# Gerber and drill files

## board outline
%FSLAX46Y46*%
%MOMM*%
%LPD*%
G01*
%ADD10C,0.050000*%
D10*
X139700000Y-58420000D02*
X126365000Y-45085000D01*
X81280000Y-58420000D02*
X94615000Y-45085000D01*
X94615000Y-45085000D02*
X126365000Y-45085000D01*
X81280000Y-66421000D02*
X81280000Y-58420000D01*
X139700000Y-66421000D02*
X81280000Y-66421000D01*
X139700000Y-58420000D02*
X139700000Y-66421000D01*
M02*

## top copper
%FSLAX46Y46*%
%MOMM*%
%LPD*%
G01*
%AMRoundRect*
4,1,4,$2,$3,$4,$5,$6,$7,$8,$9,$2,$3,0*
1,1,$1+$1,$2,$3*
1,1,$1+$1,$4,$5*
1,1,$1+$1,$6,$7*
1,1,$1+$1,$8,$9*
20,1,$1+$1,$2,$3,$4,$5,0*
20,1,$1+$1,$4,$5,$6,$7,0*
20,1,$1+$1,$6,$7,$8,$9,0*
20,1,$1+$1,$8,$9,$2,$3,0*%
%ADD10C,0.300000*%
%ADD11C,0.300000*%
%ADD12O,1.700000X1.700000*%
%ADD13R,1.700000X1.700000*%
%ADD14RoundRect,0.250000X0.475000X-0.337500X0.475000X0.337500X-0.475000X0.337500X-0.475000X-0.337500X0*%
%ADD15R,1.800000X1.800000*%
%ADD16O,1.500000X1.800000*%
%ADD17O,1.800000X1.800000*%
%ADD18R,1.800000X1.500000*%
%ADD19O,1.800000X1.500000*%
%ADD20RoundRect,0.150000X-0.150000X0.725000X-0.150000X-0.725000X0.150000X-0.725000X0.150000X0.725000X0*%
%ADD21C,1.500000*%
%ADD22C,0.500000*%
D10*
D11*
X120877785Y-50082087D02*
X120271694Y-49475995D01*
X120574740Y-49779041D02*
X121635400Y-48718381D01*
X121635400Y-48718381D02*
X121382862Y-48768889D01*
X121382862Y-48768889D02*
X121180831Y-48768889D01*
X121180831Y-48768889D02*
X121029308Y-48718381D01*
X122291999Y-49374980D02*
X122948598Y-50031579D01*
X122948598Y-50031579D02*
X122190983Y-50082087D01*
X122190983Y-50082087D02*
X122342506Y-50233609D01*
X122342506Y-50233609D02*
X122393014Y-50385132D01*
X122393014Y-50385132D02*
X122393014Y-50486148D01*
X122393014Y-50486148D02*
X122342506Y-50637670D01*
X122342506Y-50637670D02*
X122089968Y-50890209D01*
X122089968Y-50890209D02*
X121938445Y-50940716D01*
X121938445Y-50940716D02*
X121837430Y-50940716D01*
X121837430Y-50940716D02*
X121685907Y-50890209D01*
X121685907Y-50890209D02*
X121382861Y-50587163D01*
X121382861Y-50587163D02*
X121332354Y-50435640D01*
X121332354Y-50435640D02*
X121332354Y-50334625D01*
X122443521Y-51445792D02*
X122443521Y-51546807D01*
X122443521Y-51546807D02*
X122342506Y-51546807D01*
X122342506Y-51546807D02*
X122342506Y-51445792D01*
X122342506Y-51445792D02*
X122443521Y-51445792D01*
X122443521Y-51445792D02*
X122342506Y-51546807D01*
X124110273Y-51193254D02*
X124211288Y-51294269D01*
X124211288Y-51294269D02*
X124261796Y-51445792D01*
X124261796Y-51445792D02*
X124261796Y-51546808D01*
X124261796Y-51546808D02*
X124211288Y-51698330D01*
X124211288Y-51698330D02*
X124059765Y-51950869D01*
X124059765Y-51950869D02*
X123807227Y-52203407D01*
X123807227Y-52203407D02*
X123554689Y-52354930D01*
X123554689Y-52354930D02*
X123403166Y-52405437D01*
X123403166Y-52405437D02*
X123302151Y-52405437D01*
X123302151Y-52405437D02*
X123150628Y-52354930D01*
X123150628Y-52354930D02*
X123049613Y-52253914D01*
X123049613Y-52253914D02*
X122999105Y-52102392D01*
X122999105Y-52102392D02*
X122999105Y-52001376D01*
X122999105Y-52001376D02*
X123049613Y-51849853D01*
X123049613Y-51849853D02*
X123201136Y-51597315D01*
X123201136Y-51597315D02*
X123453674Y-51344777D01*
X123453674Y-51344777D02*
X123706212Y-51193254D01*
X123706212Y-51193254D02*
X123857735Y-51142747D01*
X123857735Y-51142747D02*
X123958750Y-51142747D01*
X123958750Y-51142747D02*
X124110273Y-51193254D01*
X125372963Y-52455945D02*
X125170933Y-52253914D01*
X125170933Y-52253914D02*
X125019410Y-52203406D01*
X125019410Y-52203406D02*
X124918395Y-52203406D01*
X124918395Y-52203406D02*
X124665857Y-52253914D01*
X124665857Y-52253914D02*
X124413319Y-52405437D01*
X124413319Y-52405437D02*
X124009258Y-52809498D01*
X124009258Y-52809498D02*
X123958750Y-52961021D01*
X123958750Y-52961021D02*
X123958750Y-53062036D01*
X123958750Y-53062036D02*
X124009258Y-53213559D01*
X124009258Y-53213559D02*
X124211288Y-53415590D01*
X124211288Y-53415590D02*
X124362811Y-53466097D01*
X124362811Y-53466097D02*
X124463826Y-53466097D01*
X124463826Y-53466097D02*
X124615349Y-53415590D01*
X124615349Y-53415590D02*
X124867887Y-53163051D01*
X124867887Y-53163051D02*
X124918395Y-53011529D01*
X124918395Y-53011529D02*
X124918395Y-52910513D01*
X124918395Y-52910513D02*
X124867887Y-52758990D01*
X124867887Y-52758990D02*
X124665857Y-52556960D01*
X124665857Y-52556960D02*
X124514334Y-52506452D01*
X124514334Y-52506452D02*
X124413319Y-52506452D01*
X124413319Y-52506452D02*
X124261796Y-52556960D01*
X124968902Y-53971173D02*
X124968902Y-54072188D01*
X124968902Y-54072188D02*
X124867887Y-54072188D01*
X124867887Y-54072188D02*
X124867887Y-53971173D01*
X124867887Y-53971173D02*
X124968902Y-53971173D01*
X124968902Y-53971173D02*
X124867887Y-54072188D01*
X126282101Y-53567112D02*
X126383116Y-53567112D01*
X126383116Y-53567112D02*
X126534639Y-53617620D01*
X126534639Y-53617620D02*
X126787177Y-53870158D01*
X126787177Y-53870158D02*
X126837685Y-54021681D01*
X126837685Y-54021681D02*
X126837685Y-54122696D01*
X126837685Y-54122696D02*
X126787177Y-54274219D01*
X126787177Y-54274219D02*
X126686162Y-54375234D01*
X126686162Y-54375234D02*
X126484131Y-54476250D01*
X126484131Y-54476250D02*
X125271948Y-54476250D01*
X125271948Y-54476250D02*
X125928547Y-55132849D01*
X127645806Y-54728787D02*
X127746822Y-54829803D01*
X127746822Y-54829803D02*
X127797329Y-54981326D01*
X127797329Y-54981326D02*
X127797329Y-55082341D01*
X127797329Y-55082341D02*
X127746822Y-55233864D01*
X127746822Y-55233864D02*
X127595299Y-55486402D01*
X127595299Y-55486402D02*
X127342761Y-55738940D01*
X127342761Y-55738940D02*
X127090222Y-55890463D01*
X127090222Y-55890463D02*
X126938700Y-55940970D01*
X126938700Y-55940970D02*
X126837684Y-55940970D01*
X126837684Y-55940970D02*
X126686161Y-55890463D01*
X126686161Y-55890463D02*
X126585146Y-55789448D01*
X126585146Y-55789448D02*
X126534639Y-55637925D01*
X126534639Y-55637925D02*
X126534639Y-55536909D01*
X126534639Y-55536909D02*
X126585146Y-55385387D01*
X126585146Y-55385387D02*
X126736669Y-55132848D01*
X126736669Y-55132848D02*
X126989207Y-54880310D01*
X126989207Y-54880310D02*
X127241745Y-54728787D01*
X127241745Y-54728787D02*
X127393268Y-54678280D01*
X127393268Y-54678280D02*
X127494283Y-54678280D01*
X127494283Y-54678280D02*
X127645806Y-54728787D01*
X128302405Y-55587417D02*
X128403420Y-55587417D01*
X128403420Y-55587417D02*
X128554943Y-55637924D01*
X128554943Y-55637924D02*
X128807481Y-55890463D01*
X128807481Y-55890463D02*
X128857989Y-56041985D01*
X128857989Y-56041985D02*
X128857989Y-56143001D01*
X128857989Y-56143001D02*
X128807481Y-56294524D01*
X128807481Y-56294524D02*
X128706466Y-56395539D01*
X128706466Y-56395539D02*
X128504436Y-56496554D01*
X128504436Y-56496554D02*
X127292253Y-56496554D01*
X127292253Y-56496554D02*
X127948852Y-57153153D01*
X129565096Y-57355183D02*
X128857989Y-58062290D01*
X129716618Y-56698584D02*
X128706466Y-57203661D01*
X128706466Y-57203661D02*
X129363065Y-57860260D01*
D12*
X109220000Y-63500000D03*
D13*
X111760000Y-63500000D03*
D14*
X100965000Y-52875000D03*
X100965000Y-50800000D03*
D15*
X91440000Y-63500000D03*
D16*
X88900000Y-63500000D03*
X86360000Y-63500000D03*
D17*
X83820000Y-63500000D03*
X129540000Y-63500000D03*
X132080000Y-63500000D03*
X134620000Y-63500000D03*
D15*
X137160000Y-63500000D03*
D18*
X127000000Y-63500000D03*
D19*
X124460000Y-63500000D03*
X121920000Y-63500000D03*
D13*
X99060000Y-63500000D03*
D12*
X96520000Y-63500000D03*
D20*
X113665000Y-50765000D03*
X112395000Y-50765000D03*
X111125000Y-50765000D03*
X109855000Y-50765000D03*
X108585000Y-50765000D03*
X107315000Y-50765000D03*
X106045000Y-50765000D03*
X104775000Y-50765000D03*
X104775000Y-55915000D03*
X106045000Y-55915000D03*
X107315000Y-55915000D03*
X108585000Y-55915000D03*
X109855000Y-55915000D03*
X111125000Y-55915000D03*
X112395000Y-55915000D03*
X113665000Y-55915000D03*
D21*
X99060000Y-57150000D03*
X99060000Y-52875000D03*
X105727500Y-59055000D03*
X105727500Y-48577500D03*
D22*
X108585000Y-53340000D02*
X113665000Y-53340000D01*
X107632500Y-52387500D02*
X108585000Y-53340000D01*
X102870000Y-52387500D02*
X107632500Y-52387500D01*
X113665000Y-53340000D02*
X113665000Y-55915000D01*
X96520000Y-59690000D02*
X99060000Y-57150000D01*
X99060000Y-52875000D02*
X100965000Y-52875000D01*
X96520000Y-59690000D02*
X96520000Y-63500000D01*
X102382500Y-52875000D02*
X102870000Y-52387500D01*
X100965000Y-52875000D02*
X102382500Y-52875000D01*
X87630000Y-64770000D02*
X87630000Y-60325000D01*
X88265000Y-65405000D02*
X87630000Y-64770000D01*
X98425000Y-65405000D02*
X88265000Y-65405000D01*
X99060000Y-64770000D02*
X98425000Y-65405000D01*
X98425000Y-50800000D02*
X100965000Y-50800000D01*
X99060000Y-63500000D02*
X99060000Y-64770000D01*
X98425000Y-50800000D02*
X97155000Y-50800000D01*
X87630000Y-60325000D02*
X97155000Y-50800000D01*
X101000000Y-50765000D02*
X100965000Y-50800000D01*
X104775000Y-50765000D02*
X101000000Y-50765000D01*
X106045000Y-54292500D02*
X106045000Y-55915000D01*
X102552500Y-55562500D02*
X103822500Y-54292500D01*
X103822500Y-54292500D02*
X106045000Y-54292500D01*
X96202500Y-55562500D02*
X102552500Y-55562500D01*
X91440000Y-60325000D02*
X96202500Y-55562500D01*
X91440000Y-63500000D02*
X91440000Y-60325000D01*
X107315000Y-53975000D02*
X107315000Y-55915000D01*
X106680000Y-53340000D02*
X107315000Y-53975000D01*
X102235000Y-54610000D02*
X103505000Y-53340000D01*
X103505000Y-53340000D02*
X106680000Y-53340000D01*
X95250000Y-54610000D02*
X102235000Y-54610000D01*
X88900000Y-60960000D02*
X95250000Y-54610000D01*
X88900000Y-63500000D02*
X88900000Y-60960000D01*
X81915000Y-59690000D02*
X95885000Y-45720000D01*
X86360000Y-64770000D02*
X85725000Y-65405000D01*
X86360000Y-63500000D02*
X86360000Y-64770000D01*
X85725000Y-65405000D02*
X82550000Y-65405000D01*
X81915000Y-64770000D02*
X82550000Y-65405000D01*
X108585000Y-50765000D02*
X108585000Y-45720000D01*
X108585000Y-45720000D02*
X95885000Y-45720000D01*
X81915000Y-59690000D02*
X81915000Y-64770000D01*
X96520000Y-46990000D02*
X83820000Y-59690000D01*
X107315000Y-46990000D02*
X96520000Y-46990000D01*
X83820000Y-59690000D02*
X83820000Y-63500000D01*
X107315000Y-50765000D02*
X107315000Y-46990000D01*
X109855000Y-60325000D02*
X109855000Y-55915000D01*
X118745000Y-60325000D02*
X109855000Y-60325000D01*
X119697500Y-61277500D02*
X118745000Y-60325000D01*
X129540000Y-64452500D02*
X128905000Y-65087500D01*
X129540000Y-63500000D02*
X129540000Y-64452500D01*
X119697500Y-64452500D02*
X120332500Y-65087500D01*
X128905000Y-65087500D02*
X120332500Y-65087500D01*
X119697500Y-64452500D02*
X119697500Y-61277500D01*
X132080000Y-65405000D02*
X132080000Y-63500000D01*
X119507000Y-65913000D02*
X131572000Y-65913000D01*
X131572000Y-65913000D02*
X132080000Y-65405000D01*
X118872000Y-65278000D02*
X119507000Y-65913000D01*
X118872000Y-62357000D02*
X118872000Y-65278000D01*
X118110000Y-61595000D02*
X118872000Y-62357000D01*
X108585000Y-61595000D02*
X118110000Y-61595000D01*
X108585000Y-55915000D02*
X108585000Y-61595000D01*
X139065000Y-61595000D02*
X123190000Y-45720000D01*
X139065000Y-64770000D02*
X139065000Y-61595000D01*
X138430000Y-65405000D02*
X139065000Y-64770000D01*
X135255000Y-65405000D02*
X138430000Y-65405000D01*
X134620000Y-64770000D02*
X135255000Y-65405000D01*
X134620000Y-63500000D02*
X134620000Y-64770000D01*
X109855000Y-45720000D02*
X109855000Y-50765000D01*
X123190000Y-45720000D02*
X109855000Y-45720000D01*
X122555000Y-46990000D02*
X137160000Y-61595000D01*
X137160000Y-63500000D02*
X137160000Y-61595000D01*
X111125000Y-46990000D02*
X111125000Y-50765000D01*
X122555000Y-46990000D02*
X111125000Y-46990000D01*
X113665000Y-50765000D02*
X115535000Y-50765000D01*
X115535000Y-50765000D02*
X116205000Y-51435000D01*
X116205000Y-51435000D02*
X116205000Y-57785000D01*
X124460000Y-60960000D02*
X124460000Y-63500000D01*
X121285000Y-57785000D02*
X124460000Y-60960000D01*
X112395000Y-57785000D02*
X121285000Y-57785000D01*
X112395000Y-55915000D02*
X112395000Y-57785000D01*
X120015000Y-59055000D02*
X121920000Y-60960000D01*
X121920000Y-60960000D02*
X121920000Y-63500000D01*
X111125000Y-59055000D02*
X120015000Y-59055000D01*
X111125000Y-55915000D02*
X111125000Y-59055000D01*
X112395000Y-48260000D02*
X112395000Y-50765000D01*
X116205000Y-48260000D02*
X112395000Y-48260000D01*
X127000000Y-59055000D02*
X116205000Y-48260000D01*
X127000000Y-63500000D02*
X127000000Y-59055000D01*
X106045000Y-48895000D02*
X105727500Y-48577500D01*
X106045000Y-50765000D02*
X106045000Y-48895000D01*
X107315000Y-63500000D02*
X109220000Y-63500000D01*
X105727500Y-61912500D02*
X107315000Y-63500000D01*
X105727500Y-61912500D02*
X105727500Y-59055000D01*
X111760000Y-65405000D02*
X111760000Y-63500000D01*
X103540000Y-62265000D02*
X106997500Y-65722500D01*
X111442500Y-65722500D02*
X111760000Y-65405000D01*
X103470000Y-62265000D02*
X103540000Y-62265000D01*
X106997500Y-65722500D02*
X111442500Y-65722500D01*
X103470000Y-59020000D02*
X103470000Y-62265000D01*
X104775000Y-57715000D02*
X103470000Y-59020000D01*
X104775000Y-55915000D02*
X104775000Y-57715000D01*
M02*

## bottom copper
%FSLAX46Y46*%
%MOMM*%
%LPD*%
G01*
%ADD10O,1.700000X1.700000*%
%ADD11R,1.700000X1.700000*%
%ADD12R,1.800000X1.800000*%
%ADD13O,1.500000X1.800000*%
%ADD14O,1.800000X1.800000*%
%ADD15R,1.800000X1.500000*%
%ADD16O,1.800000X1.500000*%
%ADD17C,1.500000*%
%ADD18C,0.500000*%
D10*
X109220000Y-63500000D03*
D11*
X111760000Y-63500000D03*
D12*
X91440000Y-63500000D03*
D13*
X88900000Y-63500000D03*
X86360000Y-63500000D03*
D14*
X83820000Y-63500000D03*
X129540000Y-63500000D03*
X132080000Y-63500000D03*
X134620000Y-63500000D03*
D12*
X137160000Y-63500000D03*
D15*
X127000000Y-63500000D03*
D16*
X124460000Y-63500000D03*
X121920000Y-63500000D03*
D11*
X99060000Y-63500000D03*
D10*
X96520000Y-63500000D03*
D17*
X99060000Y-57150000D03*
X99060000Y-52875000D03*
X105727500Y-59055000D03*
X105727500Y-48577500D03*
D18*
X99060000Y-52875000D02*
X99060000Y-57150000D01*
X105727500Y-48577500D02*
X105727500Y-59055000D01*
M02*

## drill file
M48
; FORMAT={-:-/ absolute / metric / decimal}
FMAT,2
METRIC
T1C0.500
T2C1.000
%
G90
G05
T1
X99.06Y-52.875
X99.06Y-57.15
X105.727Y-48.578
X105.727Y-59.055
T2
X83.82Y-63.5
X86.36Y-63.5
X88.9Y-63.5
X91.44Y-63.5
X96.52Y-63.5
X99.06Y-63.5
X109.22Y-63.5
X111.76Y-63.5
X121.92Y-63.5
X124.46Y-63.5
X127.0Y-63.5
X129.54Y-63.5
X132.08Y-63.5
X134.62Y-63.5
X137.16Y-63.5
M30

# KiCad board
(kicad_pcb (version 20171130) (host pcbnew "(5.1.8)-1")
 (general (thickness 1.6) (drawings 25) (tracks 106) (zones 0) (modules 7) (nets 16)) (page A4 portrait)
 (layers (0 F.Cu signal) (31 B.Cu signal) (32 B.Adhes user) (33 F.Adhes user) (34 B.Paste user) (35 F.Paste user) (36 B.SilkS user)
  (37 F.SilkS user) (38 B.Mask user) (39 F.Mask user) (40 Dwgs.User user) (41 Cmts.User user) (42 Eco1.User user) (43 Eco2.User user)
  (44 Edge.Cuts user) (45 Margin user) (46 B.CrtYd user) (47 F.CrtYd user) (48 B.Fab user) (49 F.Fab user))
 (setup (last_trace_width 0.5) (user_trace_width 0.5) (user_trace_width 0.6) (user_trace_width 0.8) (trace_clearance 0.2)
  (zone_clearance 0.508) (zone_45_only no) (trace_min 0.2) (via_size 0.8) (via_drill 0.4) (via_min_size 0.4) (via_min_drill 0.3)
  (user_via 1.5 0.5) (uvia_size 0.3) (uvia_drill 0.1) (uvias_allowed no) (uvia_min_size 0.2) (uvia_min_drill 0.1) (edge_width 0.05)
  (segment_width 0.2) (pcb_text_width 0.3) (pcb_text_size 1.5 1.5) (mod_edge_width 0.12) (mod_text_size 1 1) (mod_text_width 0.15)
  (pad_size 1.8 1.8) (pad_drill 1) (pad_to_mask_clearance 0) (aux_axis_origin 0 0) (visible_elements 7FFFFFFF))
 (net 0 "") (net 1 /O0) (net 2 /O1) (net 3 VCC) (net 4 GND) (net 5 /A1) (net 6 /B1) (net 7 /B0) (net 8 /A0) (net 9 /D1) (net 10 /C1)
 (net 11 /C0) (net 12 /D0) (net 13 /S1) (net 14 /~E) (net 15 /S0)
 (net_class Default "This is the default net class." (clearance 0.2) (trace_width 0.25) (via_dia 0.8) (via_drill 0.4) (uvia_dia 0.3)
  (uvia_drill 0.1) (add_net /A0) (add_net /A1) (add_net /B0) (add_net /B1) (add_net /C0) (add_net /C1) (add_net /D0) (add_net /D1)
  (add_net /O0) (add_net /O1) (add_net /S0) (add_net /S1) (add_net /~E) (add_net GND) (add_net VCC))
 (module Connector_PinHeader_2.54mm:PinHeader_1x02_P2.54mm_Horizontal (layer F.Cu) (at 111.76 63.5 270)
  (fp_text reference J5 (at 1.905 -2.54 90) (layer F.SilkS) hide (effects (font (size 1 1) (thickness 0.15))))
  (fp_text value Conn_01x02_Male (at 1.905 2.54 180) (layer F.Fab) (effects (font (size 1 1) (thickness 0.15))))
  (pad 2 thru_hole oval (at 0 2.54 270) (size 1.7 1.7) (drill 1) (layers *.Cu *.Mask) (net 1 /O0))
  (pad 1 thru_hole rect (at 0 0 270) (size 1.7 1.7) (drill 1) (layers *.Cu *.Mask) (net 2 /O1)))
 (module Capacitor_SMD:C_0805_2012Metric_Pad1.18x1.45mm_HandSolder (layer F.Cu) (at 100.965 51.8375 90)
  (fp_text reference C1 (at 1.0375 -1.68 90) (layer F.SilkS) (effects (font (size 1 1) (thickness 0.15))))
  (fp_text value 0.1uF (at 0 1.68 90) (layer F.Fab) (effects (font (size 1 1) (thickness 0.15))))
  (pad 1 smd roundrect (at -1.0375 0 90) (size 1.175 1.45) (layers F.Cu F.Paste F.Mask) (roundrect_rratio 0.2127659574468085) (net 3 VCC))
  (pad 2 smd roundrect (at 1.0375 0 90) (size 1.175 1.45) (layers F.Cu F.Paste F.Mask) (roundrect_rratio 0.2127659574468085) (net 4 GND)))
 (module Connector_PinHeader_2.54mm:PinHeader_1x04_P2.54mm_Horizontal (layer F.Cu) (at 91.44 63.5 270)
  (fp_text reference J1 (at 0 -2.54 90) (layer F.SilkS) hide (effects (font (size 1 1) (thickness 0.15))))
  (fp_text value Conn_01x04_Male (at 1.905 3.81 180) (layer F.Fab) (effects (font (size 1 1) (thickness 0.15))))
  (pad 1 thru_hole rect (at 0 0 270) (size 1.8 1.8) (drill 1) (layers *.Cu *.Mask) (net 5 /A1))
  (pad 2 thru_hole oval (at 0 2.54 270) (size 1.8 1.5) (drill 1) (layers *.Cu *.Mask) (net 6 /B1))
  (pad 3 thru_hole oval (at 0 5.08 270) (size 1.8 1.5) (drill 1) (layers *.Cu *.Mask) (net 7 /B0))
  (pad 4 thru_hole oval (at 0 7.62 270) (size 1.8 1.8) (drill 1) (layers *.Cu *.Mask) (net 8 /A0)))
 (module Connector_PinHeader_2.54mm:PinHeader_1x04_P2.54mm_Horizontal (layer F.Cu) (at 137.16 63.5 270)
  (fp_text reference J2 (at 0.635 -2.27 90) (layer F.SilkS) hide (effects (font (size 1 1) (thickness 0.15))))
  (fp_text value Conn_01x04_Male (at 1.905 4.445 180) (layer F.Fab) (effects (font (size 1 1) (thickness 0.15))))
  (pad 4 thru_hole oval (at 0 7.62 270) (size 1.8 1.8) (drill 1) (layers *.Cu *.Mask) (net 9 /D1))
  (pad 3 thru_hole oval (at 0 5.08 270) (size 1.8 1.8) (drill 1) (layers *.Cu *.Mask) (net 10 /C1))
  (pad 2 thru_hole oval (at 0 2.54 270) (size 1.8 1.8) (drill 1) (layers *.Cu *.Mask) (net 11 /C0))
  (pad 1 thru_hole rect (at 0 0 270) (size 1.8 1.8) (drill 1) (layers *.Cu *.Mask) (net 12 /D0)))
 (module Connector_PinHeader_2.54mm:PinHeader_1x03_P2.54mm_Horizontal (layer F.Cu) (at 127 63.5 270)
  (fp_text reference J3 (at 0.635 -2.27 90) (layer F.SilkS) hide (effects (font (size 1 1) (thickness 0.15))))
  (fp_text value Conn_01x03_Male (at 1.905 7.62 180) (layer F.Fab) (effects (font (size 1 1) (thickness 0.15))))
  (pad 1 thru_hole rect (at 0 0 270) (size 1.5 1.8) (drill 1) (layers *.Cu *.Mask) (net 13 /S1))
  (pad 2 thru_hole oval (at 0 2.54 270) (size 1.5 1.8) (drill 1) (layers *.Cu *.Mask) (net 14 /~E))
  (pad 3 thru_hole oval (at 0 5.08 270) (size 1.5 1.8) (drill 1) (layers *.Cu *.Mask) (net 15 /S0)))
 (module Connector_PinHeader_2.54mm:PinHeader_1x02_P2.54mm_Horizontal (layer F.Cu) (at 99.06 63.5 270)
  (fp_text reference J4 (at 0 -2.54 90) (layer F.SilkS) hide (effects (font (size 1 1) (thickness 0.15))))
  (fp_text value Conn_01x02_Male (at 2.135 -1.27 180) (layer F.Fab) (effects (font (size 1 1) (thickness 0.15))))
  (pad 1 thru_hole rect (at 0 0 270) (size 1.7 1.7) (drill 1) (layers *.Cu *.Mask) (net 4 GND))
  (pad 2 thru_hole oval (at 0 2.54 270) (size 1.7 1.7) (drill 1) (layers *.Cu *.Mask) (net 3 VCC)))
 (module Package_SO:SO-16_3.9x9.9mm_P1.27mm (layer F.Cu) (at 109.22 53.34 270)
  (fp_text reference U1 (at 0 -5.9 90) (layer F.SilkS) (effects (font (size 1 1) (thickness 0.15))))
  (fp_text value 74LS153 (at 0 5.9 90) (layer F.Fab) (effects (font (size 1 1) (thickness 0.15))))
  (pad 1 smd roundrect (at -2.575 -4.445 270) (size 1.75 0.6) (layers F.Cu F.Paste F.Mask) (roundrect_rratio 0.25) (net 14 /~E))
  (pad 2 smd roundrect (at -2.575 -3.175 270) (size 1.75 0.6) (layers F.Cu F.Paste F.Mask) (roundrect_rratio 0.25) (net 13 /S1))
  (pad 3 smd roundrect (at -2.575 -1.905 270) (size 1.75 0.6) (layers F.Cu F.Paste F.Mask) (roundrect_rratio 0.25) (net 12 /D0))
  (pad 4 smd roundrect (at -2.575 -0.635 270) (size 1.75 0.6) (layers F.Cu F.Paste F.Mask) (roundrect_rratio 0.25) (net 11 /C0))
  (pad 5 smd roundrect (at -2.575 0.635 270) (size 1.75 0.6) (layers F.Cu F.Paste F.Mask) (roundrect_rratio 0.25) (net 7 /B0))
  (pad 6 smd roundrect (at -2.575 1.905 270) (size 1.75 0.6) (layers F.Cu F.Paste F.Mask) (roundrect_rratio 0.25) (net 8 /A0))
  (pad 7 smd roundrect (at -2.575 3.175 270) (size 1.75 0.6) (layers F.Cu F.Paste F.Mask) (roundrect_rratio 0.25) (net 1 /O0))
  (pad 8 smd roundrect (at -2.575 4.445 270) (size 1.75 0.6) (layers F.Cu F.Paste F.Mask) (roundrect_rratio 0.25) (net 4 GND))
  (pad 9 smd roundrect (at 2.575 4.445 270) (size 1.75 0.6) (layers F.Cu F.Paste F.Mask) (roundrect_rratio 0.25) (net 2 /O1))
  (pad 10 smd roundrect (at 2.575 3.175 270) (size 1.75 0.6) (layers F.Cu F.Paste F.Mask) (roundrect_rratio 0.25) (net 5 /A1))
  (pad 11 smd roundrect (at 2.575 1.905 270) (size 1.75 0.6) (layers F.Cu F.Paste F.Mask) (roundrect_rratio 0.25) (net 6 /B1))
  (pad 12 smd roundrect (at 2.575 0.635 270) (size 1.75 0.6) (layers F.Cu F.Paste F.Mask) (roundrect_rratio 0.25) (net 10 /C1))
  (pad 13 smd roundrect (at 2.575 -0.635 270) (size 1.75 0.6) (layers F.Cu F.Paste F.Mask) (roundrect_rratio 0.25) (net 9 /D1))
  (pad 14 smd roundrect (at 2.575 -1.905 270) (size 1.75 0.6) (layers F.Cu F.Paste F.Mask) (roundrect_rratio 0.25) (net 15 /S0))
  (pad 15 smd roundrect (at 2.575 -3.175 270) (size 1.75 0.6) (layers F.Cu F.Paste F.Mask) (roundrect_rratio 0.25) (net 14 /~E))
  (pad 16 smd roundrect (at 2.575 -4.445 270) (size 1.75 0.6) (layers F.Cu F.Paste F.Mask) (roundrect_rratio 0.25) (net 3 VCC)))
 (gr_line (start 139.7 58.42) (end 126.365 45.085) (layer Edge.Cuts) (width 0.05))
 (gr_line (start 81.28 58.42) (end 94.615 45.085) (layer Edge.Cuts) (width 0.05))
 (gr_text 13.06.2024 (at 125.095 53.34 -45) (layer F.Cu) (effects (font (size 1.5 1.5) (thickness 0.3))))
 (gr_line (start 94.615 45.085) (end 126.365 45.085) (layer Edge.Cuts) (width 0.05))
 (gr_line (start 81.28 66.421) (end 81.28 58.42) (layer Edge.Cuts) (width 0.05))
 (gr_line (start 139.7 66.421) (end 81.28 66.421) (layer Edge.Cuts) (width 0.05))
 (gr_line (start 139.7 58.42) (end 139.7 66.421) (layer Edge.Cuts) (width 0.05))
 (segment (start 108.585 53.34) (end 113.665 53.34) (width 0.5) (layer F.Cu) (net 3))
 (segment (start 107.6325 52.3875) (end 108.585 53.34) (width 0.5) (layer F.Cu) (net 3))
 (segment (start 102.87 52.3875) (end 107.6325 52.3875) (width 0.5) (layer F.Cu) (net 3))
 (via (at 99.06 57.15) (size 1.5) (drill 0.5) (layers F.Cu B.Cu) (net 3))
 (via (at 99.06 52.875) (size 1.5) (drill 0.5) (layers F.Cu B.Cu) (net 3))
 (segment (start 99.06 52.875) (end 99.06 57.15) (width 0.5) (layer B.Cu) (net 3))
 (segment (start 113.665 53.34) (end 113.665 55.915) (width 0.5) (layer F.Cu) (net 3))
 (segment (start 96.52 59.69) (end 99.06 57.15) (width 0.5) (layer F.Cu) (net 3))
 (segment (start 99.06 52.875) (end 100.965 52.875) (width 0.5) (layer F.Cu) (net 3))
 (segment (start 96.52 59.69) (end 96.52 63.5) (width 0.5) (layer F.Cu) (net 3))
 (segment (start 102.3825 52.875) (end 102.87 52.3875) (width 0.5) (layer F.Cu) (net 3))
 (segment (start 100.965 52.875) (end 102.3825 52.875) (width 0.5) (layer F.Cu) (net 3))
 (segment (start 87.63 64.77) (end 87.63 60.325) (width 0.5) (layer F.Cu) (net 4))
 (segment (start 88.265 65.405) (end 87.63 64.77) (width 0.5) (layer F.Cu) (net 4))
 (segment (start 98.425 65.405) (end 88.265 65.405) (width 0.5) (layer F.Cu) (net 4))
 (segment (start 99.06 64.77) (end 98.425 65.405) (width 0.5) (layer F.Cu) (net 4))
 (segment (start 98.425 50.8) (end 100.965 50.8) (width 0.5) (layer F.Cu) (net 4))
 (segment (start 99.06 63.5) (end 99.06 64.77) (width 0.5) (layer F.Cu) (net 4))
 (segment (start 98.425 50.8) (end 97.155 50.8) (width 0.5) (layer F.Cu) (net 4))
 (segment (start 87.63 60.325) (end 97.155 50.8) (width 0.5) (layer F.Cu) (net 4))
 (segment (start 101 50.765) (end 100.965 50.8) (width 0.5) (layer F.Cu) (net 4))
 (segment (start 104.775 50.765) (end 101 50.765) (width 0.5) (layer F.Cu) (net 4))
 (segment (start 106.045 54.2925) (end 106.045 55.915) (width 0.5) (layer F.Cu) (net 5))
 (segment (start 102.5525 55.5625) (end 103.8225 54.2925) (width 0.5) (layer F.Cu) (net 5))
 (segment (start 103.8225 54.2925) (end 106.045 54.2925) (width 0.5) (layer F.Cu) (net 5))
 (segment (start 96.2025 55.5625) (end 102.5525 55.5625) (width 0.5) (layer F.Cu) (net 5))
 (segment (start 91.44 60.325) (end 96.2025 55.5625) (width 0.5) (layer F.Cu) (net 5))
 (segment (start 91.44 63.5) (end 91.44 60.325) (width 0.5) (layer F.Cu) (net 5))
 (segment (start 107.315 53.975) (end 107.315 55.915) (width 0.5) (layer F.Cu) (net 6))
 (segment (start 106.68 53.34) (end 107.315 53.975) (width 0.5) (layer F.Cu) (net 6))
 (segment (start 102.235 54.61) (end 103.505 53.34) (width 0.5) (layer F.Cu) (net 6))
 (segment (start 103.505 53.34) (end 106.68 53.34) (width 0.5) (layer F.Cu) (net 6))
 (segment (start 95.25 54.61) (end 102.235 54.61) (width 0.5) (layer F.Cu) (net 6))
 (segment (start 88.9 60.96) (end 95.25 54.61) (width 0.5) (layer F.Cu) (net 6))
 (segment (start 88.9 63.5) (end 88.9 60.96) (width 0.5) (layer F.Cu) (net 6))
 (segment (start 81.915 59.69) (end 95.885 45.72) (width 0.5) (layer F.Cu) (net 7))
 (segment (start 86.36 64.77) (end 85.725 65.405) (width 0.5) (layer F.Cu) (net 7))
 (segment (start 86.36 63.5) (end 86.36 64.77) (width 0.5) (layer F.Cu) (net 7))
 (segment (start 85.725 65.405) (end 82.55 65.405) (width 0.5) (layer F.Cu) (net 7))
 (segment (start 81.915 64.77) (end 82.55 65.405) (width 0.5) (layer F.Cu) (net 7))
 (segment (start 108.585 50.765) (end 108.585 45.72) (width 0.5) (layer F.Cu) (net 7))
 (segment (start 108.585 45.72) (end 95.885 45.72) (width 0.5) (layer F.Cu) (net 7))
 (segment (start 81.915 59.69) (end 81.915 64.77) (width 0.5) (layer F.Cu) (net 7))
 (segment (start 96.52 46.99) (end 83.82 59.69) (width 0.5) (layer F.Cu) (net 8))
 (segment (start 107.315 46.99) (end 96.52 46.99) (width 0.5) (layer F.Cu) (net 8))
 (segment (start 83.82 59.69) (end 83.82 63.5) (width 0.5) (layer F.Cu) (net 8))
 (segment (start 107.315 50.765) (end 107.315 46.99) (width 0.5) (layer F.Cu) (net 8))
 (segment (start 109.855 60.325) (end 109.855 55.915) (width 0.5) (layer F.Cu) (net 9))
 (segment (start 118.745 60.325) (end 109.855 60.325) (width 0.5) (layer F.Cu) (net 9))
 (segment (start 119.6975 61.2775) (end 118.745 60.325) (width 0.5) (layer F.Cu) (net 9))
 (segment (start 129.54 64.4525) (end 128.905 65.0875) (width 0.5) (layer F.Cu) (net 9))
 (segment (start 129.54 63.5) (end 129.54 64.4525) (width 0.5) (layer F.Cu) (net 9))
 (segment (start 119.6975 64.4525) (end 120.3325 65.0875) (width 0.5) (layer F.Cu) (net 9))
 (segment (start 128.905 65.0875) (end 120.3325 65.0875) (width 0.5) (layer F.Cu) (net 9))
 (segment (start 119.6975 64.4525) (end 119.6975 61.2775) (width 0.5) (layer F.Cu) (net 9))
 (segment (start 132.08 65.405) (end 132.08 63.5) (width 0.5) (layer F.Cu) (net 10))
 (segment (start 119.507 65.913) (end 131.572 65.913) (width 0.5) (layer F.Cu) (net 10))
 (segment (start 131.572 65.913) (end 132.08 65.405) (width 0.5) (layer F.Cu) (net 10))
 (segment (start 118.872 65.278) (end 119.507 65.913) (width 0.5) (layer F.Cu) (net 10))
 (segment (start 118.872 62.357) (end 118.872 65.278) (width 0.5) (layer F.Cu) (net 10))
 (segment (start 118.11 61.595) (end 118.872 62.357) (width 0.5) (layer F.Cu) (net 10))
 (segment (start 108.585 61.595) (end 118.11 61.595) (width 0.5) (layer F.Cu) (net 10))
 (segment (start 108.585 55.915) (end 108.585 61.595) (width 0.5) (layer F.Cu) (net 10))
 (segment (start 139.065 61.595) (end 123.19 45.72) (width 0.5) (layer F.Cu) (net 11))
 (segment (start 139.065 64.77) (end 139.065 61.595) (width 0.5) (layer F.Cu) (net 11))
 (segment (start 138.43 65.405) (end 139.065 64.77) (width 0.5) (layer F.Cu) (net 11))
 (segment (start 135.255 65.405) (end 138.43 65.405) (width 0.5) (layer F.Cu) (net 11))
 (segment (start 134.62 64.77) (end 135.255 65.405) (width 0.5) (layer F.Cu) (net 11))
 (segment (start 134.62 63.5) (end 134.62 64.77) (width 0.5) (layer F.Cu) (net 11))
 (segment (start 109.855 45.72) (end 109.855 50.765) (width 0.5) (layer F.Cu) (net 11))
 (segment (start 123.19 45.72) (end 109.855 45.72) (width 0.5) (layer F.Cu) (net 11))
 (segment (start 122.555 46.99) (end 137.16 61.595) (width 0.5) (layer F.Cu) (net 12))
 (segment (start 137.16 63.5) (end 137.16 61.595) (width 0.5) (layer F.Cu) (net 12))
 (segment (start 111.125 46.99) (end 111.125 50.765) (width 0.5) (layer F.Cu) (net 12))
 (segment (start 122.555 46.99) (end 111.125 46.99) (width 0.5) (layer F.Cu) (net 12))
 (segment (start 113.665 50.765) (end 115.535 50.765) (width 0.5) (layer F.Cu) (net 14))
 (segment (start 115.535 50.765) (end 116.205 51.435) (width 0.5) (layer F.Cu) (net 14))
 (segment (start 116.205 51.435) (end 116.205 57.785) (width 0.5) (layer F.Cu) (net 14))
 (segment (start 124.46 60.96) (end 124.46 63.5) (width 0.5) (layer F.Cu) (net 14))
 (segment (start 121.285 57.785) (end 124.46 60.96) (width 0.5) (layer F.Cu) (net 14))
 (segment (start 112.395 57.785) (end 121.285 57.785) (width 0.5) (layer F.Cu) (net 14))
 (segment (start 112.395 55.915) (end 112.395 57.785) (width 0.5) (layer F.Cu) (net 14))
 (segment (start 120.015 59.055) (end 121.92 60.96) (width 0.5) (layer F.Cu) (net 15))
 (segment (start 121.92 60.96) (end 121.92 63.5) (width 0.5) (layer F.Cu) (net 15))
 (segment (start 111.125 59.055) (end 120.015 59.055) (width 0.5) (layer F.Cu) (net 15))
 (segment (start 111.125 55.915) (end 111.125 59.055) (width 0.5) (layer F.Cu) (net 15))
 (segment (start 112.395 48.26) (end 112.395 50.765) (width 0.5) (layer F.Cu) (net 13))
 (segment (start 116.205 48.26) (end 112.395 48.26) (width 0.5) (layer F.Cu) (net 13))
 (segment (start 127 59.055) (end 116.205 48.26) (width 0.5) (layer F.Cu) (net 13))
 (segment (start 127 63.5) (end 127 59.055) (width 0.5) (layer F.Cu) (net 13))
 (via (at 105.7275 59.055) (size 1.5) (drill 0.5) (layers F.Cu B.Cu) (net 1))
 (via (at 105.7275 48.5775) (size 1.5) (drill 0.5) (layers F.Cu B.Cu) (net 1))
 (segment (start 105.7275 48.5775) (end 105.7275 59.055) (width 0.5) (layer B.Cu) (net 1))
 (segment (start 106.045 48.895) (end 105.7275 48.5775) (width 0.5) (layer F.Cu) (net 1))
 (segment (start 106.045 50.765) (end 106.045 48.895) (width 0.5) (layer F.Cu) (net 1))
 (segment (start 107.315 63.5) (end 109.22 63.5) (width 0.5) (layer F.Cu) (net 1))
 (segment (start 105.7275 61.9125) (end 107.315 63.5) (width 0.5) (layer F.Cu) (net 1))
 (segment (start 105.7275 61.9125) (end 105.7275 59.055) (width 0.5) (layer F.Cu) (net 1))
 (segment (start 111.76 65.405) (end 111.76 63.5) (width 0.5) (layer F.Cu) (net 2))
 (segment (start 103.54 62.265) (end 106.9975 65.7225) (width 0.5) (layer F.Cu) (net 2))
 (segment (start 111.4425 65.7225) (end 111.76 65.405) (width 0.5) (layer F.Cu) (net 2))
 (segment (start 103.47 62.265) (end 103.54 62.265) (width 0.5) (layer F.Cu) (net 2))
 (segment (start 106.9975 65.7225) (end 111.4425 65.7225) (width 0.5) (layer F.Cu) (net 2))
 (segment (start 103.47 59.02) (end 103.47 62.265) (width 0.5) (layer F.Cu) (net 2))
 (segment (start 104.775 57.715) (end 103.47 59.02) (width 0.5) (layer F.Cu) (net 2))
 (segment (start 104.775 55.915) (end 104.775 57.715) (width 0.5) (layer F.Cu) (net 2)))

